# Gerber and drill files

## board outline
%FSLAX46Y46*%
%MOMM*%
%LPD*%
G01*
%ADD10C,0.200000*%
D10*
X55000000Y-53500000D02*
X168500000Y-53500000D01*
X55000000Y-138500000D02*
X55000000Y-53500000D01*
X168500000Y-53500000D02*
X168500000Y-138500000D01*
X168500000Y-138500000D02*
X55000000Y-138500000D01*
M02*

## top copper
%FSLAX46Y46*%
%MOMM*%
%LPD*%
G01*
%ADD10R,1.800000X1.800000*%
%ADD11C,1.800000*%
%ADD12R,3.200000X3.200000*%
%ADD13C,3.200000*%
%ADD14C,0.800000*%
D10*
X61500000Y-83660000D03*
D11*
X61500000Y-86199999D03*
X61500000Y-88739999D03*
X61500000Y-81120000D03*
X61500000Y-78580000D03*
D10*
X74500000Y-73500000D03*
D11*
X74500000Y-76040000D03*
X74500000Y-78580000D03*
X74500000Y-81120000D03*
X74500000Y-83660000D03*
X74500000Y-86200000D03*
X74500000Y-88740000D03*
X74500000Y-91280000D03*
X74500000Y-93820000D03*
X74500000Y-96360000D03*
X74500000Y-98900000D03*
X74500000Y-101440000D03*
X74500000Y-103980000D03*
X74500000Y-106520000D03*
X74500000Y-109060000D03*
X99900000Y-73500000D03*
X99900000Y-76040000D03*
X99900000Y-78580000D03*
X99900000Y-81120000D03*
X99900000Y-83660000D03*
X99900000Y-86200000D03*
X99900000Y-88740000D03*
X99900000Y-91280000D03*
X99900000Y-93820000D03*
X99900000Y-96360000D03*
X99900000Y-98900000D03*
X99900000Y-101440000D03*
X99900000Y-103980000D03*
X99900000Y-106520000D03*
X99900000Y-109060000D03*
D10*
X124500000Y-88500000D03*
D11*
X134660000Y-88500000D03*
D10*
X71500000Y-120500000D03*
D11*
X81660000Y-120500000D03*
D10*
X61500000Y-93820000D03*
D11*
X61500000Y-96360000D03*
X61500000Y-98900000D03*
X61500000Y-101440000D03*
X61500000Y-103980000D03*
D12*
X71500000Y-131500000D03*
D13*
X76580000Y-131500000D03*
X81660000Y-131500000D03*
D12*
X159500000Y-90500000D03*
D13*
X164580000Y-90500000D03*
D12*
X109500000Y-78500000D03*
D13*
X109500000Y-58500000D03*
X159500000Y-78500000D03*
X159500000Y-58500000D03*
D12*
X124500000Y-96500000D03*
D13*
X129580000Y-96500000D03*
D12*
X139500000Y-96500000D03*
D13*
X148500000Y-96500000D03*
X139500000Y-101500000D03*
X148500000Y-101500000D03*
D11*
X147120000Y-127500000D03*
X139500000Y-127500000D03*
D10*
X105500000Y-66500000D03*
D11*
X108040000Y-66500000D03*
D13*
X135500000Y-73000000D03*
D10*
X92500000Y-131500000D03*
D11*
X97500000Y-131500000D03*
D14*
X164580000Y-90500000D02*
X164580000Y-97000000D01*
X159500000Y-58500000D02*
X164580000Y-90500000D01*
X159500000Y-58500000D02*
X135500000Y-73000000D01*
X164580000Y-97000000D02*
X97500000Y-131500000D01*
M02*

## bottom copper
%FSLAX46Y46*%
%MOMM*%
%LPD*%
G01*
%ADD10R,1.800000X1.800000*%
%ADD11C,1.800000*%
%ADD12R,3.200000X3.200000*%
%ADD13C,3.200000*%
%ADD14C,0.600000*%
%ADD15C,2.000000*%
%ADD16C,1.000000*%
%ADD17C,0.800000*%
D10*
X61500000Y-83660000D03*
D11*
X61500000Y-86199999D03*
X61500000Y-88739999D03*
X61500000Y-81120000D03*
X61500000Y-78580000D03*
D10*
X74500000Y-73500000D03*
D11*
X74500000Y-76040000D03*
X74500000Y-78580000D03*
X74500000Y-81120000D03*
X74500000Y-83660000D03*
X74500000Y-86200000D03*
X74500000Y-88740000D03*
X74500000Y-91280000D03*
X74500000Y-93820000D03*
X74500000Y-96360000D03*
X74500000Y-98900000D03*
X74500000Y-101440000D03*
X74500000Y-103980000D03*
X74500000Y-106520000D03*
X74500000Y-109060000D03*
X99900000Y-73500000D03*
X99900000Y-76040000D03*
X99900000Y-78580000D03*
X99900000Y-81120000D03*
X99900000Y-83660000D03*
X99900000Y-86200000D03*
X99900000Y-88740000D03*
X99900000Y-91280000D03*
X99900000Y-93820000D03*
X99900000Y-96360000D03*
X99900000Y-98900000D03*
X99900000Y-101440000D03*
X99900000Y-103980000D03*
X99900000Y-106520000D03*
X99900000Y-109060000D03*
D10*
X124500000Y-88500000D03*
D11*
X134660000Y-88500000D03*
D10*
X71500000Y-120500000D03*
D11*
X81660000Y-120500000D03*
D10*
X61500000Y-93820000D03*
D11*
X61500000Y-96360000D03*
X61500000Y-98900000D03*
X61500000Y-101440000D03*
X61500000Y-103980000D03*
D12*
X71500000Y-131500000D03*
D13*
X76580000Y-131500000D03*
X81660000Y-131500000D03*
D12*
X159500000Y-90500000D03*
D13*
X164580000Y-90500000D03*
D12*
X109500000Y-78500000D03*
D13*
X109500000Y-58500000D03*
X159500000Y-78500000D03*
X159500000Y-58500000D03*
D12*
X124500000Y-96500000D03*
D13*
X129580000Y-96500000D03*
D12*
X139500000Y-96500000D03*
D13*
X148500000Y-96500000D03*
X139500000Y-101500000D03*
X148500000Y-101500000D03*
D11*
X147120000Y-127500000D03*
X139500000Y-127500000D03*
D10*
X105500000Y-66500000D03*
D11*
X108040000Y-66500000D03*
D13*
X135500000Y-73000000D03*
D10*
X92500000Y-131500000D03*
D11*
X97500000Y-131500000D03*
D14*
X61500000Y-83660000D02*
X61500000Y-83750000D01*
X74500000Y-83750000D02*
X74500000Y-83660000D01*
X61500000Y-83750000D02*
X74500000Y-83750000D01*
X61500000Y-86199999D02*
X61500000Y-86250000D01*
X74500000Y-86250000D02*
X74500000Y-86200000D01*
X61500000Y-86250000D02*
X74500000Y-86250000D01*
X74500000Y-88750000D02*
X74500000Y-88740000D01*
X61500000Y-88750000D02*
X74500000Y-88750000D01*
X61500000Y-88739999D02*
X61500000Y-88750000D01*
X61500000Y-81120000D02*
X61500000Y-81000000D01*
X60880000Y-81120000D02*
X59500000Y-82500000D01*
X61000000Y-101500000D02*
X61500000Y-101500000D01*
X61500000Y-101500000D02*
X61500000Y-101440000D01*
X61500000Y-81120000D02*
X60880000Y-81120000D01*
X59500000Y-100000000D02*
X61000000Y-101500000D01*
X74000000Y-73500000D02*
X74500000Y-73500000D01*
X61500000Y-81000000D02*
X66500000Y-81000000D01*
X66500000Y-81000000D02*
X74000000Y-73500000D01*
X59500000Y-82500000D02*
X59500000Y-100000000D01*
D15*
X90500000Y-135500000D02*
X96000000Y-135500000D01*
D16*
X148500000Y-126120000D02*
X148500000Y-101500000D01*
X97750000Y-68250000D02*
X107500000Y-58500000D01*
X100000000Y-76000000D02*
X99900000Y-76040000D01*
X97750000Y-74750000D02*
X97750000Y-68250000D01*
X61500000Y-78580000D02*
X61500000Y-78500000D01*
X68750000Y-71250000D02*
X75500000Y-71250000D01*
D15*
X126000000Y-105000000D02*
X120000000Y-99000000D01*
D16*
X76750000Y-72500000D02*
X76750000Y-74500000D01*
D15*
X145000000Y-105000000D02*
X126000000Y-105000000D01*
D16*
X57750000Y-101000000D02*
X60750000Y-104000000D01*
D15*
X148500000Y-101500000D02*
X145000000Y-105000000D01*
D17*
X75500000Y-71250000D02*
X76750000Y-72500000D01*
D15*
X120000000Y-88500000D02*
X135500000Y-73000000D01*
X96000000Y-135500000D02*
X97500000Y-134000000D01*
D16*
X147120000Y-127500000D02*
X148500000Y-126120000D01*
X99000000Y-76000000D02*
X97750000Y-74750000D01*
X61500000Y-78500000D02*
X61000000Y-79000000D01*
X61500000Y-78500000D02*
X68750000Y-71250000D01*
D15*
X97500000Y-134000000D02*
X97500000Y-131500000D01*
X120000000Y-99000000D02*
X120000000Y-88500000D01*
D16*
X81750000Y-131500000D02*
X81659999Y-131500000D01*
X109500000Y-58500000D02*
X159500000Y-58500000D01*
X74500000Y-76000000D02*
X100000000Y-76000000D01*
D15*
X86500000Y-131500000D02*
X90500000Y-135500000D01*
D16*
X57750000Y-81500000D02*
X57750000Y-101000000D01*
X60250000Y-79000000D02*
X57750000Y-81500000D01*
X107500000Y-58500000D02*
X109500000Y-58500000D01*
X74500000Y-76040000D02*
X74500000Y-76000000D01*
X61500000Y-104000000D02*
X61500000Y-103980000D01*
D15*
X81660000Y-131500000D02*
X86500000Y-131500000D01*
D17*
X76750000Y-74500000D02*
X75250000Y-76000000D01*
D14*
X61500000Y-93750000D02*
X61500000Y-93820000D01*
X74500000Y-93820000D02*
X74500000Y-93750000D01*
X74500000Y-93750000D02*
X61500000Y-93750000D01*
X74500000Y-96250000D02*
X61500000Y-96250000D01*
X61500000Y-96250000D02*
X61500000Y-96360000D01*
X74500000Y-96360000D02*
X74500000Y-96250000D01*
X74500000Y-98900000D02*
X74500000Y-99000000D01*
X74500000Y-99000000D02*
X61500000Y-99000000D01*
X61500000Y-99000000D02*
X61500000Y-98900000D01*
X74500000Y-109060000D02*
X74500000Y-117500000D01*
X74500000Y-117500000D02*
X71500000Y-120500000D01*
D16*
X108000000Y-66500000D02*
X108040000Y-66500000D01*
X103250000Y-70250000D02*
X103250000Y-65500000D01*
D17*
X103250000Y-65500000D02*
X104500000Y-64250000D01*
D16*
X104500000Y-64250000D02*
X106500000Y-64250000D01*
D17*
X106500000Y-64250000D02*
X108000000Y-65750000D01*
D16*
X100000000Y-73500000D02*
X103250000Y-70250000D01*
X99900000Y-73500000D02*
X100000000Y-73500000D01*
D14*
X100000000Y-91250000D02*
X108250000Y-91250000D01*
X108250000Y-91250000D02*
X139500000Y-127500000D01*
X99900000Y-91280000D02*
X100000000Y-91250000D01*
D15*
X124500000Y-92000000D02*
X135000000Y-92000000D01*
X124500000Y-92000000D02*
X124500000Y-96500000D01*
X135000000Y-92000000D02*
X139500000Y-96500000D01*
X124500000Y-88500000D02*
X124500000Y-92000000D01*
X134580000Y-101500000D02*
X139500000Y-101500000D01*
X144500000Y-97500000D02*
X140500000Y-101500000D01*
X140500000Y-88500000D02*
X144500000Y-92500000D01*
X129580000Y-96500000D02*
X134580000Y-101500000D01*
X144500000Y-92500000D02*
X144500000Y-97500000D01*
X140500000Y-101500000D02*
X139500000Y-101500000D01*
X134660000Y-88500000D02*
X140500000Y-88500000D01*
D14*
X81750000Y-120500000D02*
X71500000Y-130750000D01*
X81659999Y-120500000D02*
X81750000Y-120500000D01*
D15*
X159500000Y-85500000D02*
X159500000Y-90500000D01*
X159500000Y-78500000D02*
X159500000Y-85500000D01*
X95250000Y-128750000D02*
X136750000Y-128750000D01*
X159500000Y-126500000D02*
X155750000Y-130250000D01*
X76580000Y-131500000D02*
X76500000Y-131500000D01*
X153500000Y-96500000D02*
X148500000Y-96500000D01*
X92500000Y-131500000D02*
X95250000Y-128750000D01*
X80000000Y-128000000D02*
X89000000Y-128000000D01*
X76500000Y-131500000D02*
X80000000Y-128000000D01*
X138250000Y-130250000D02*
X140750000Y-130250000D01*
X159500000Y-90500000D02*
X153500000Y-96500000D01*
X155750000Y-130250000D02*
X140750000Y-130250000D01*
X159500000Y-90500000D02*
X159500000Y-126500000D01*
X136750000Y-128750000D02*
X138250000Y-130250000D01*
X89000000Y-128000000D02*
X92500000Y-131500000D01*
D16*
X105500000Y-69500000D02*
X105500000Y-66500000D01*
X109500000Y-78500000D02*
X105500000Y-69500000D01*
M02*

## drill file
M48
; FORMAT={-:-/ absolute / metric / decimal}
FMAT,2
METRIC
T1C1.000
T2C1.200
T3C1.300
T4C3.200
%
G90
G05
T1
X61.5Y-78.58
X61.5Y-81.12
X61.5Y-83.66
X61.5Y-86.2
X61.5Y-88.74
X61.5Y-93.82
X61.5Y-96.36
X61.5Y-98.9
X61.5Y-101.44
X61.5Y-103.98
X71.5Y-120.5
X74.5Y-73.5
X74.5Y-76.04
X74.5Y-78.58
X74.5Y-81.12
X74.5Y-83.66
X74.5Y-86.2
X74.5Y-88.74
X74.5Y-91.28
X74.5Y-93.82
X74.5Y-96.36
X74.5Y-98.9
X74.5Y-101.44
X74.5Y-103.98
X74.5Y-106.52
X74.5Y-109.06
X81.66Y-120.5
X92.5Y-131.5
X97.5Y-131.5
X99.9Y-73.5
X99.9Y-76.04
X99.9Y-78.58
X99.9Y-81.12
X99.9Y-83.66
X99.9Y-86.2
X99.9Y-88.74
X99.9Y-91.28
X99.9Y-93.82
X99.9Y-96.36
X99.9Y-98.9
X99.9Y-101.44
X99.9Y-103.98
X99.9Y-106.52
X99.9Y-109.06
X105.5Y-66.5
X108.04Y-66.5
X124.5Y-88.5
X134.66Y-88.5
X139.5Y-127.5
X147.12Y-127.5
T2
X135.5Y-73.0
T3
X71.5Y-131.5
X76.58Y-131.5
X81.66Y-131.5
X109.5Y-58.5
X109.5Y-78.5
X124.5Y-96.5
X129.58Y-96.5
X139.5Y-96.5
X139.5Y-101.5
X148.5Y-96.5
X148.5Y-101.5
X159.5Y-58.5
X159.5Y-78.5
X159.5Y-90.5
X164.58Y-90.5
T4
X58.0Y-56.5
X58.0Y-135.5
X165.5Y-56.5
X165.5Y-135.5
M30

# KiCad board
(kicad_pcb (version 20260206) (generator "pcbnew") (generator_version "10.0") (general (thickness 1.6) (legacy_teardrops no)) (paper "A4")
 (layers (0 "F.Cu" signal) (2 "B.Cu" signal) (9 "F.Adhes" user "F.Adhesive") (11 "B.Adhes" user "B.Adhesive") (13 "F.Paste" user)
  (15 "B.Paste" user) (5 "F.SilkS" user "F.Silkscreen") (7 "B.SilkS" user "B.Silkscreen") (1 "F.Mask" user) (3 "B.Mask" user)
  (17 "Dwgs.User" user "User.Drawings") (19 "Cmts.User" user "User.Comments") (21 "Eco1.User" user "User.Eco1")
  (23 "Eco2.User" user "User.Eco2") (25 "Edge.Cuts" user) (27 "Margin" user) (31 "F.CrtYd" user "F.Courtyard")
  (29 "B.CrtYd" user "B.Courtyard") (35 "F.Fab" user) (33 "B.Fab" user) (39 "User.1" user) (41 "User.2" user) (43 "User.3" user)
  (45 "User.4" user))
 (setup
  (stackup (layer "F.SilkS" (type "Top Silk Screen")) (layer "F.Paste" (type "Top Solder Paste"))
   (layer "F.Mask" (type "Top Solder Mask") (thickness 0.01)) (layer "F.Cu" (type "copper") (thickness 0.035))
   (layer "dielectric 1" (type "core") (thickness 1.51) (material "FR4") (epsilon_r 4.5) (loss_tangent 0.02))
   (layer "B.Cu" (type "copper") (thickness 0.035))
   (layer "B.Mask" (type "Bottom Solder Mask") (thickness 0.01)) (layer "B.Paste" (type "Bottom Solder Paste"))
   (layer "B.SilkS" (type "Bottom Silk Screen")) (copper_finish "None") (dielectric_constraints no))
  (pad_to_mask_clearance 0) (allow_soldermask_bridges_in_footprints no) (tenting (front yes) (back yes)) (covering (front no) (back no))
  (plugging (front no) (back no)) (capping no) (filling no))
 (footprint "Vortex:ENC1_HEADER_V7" (layer "F.Cu") (at 61.5 83.5 -90)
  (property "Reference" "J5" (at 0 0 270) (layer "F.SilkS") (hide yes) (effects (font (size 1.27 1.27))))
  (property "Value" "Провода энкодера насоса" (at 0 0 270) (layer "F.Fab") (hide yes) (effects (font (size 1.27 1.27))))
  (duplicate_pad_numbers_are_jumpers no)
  (pad "1" thru_hole rect (at 0.16 0 270) (size 1.8 1.8) (drill 1) (layers "*.Cu") (remove_unused_layers no) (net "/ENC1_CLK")
   (thermal_bridge_angle 45))
  (pad "2" thru_hole circle (at 2.699999 0 270) (size 1.8 1.8) (drill 1) (layers "*.Cu") (remove_unused_layers no) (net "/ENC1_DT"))
  (pad "3" thru_hole circle (at 5.239999 0 270) (size 1.8 1.8) (drill 1) (layers "*.Cu") (remove_unused_layers no) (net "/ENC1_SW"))
  (pad "4" thru_hole circle (at -2.38 0 270) (size 1.8 1.8) (drill 1) (layers "*.Cu") (remove_unused_layers no) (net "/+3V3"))
  (pad "5" thru_hole circle (at -4.92 0 270) (size 1.8 1.8) (drill 1) (layers "*.Cu") (remove_unused_layers no) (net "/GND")))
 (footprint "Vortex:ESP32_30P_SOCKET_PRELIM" (layer "F.Cu") (at 74.5 73.5)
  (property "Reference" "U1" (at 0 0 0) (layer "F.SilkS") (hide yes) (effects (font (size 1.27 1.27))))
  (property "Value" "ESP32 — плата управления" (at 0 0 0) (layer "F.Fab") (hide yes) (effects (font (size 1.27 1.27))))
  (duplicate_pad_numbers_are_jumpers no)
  (pad "1" thru_hole rect (at 0 0) (size 1.8 1.8) (drill 1) (layers "*.Cu") (remove_unused_layers no) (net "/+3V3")
   (thermal_bridge_angle 45))
  (pad "2" thru_hole circle (at 0 2.54) (size 1.8 1.8) (drill 1) (layers "*.Cu") (remove_unused_layers no) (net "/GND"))
  (pad "3" thru_hole circle (at 0 5.08) (size 1.8 1.8) (drill 1) (layers "*.Cu") (remove_unused_layers no) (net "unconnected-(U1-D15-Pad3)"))
  (pad "4" thru_hole circle (at 0 7.62) (size 1.8 1.8) (drill 1) (layers "*.Cu") (remove_unused_layers no) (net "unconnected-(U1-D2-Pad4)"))
  (pad "5" thru_hole circle (at 0 10.16) (size 1.8 1.8) (drill 1) (layers "*.Cu") (remove_unused_layers no) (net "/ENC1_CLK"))
  (pad "6" thru_hole circle (at 0 12.7) (size 1.8 1.8) (drill 1) (layers "*.Cu") (remove_unused_layers no) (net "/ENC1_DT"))
  (pad "7" thru_hole circle (at 0 15.24) (size 1.8 1.8) (drill 1) (layers "*.Cu") (remove_unused_layers no) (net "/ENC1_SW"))
  (pad "8" thru_hole circle (at 0 17.78) (size 1.8 1.8) (drill 1) (layers "*.Cu") (remove_unused_layers no) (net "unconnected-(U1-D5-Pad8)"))
  (pad "9" thru_hole circle (at 0 20.32) (size 1.8 1.8) (drill 1) (layers "*.Cu") (remove_unused_layers no) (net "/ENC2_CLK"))
  (pad "10" thru_hole circle (at 0 22.86) (size 1.8 1.8) (drill 1) (layers "*.Cu") (remove_unused_layers no) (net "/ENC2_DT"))
  (pad "11" thru_hole circle (at 0 25.4) (size 1.8 1.8) (drill 1) (layers "*.Cu") (remove_unused_layers no) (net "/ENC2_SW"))
  (pad "12" thru_hole circle (at 0 27.94) (size 1.8 1.8) (drill 1) (layers "*.Cu") (remove_unused_layers no)
   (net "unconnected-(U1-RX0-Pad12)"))
  (pad "13" thru_hole circle (at 0 30.48) (size 1.8 1.8) (drill 1) (layers "*.Cu") (remove_unused_layers no)
   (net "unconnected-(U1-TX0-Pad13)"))
  (pad "14" thru_hole circle (at 0 33.02) (size 1.8 1.8) (drill 1) (layers "*.Cu") (remove_unused_layers no)
   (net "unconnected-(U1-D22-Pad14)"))
  (pad "15" thru_hole circle (at 0 35.56) (size 1.8 1.8) (drill 1) (layers "*.Cu") (remove_unused_layers no) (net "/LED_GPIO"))
  (pad "16" thru_hole circle (at 25.4 0) (size 1.8 1.8) (drill 1) (layers "*.Cu") (remove_unused_layers no) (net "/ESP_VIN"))
  (pad "17" thru_hole circle (at 25.4 2.54) (size 1.8 1.8) (drill 1) (layers "*.Cu") (remove_unused_layers no) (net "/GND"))
  (pad "18" thru_hole circle (at 25.4 5.08) (size 1.8 1.8) (drill 1) (layers "*.Cu") (remove_unused_layers no)
   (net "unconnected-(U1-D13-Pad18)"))
  (pad "19" thru_hole circle (at 25.4 7.62) (size 1.8 1.8) (drill 1) (layers "*.Cu") (remove_unused_layers no)
   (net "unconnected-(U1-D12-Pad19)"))
  (pad "20" thru_hole circle (at 25.4 10.16) (size 1.8 1.8) (drill 1) (layers "*.Cu") (remove_unused_layers no)
   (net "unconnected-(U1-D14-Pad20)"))
  (pad "21" thru_hole circle (at 25.4 12.7) (size 1.8 1.8) (drill 1) (layers "*.Cu") (remove_unused_layers no)
   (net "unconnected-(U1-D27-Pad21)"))
  (pad "22" thru_hole circle (at 25.4 15.24) (size 1.8 1.8) (drill 1) (layers "*.Cu") (remove_unused_layers no)
   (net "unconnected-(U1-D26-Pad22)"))
  (pad "23" thru_hole circle (at 25.4 17.78) (size 1.8 1.8) (drill 1) (layers "*.Cu") (remove_unused_layers no) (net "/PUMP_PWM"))
  (pad "24" thru_hole circle (at 25.4 20.32) (size 1.8 1.8) (drill 1) (layers "*.Cu") (remove_unused_layers no)
   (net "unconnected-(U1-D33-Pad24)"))
  (pad "25" thru_hole circle (at 25.4 22.86) (size 1.8 1.8) (drill 1) (layers "*.Cu") (remove_unused_layers no)
   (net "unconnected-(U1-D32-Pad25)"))
  (pad "26" thru_hole circle (at 25.4 25.4) (size 1.8 1.8) (drill 1) (layers "*.Cu") (remove_unused_layers no)
   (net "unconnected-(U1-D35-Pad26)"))
  (pad "27" thru_hole circle (at 25.4 27.94) (size 1.8 1.8) (drill 1) (layers "*.Cu") (remove_unused_layers no)
   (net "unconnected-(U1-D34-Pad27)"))
  (pad "28" thru_hole circle (at 25.4 30.48) (size 1.8 1.8) (drill 1) (layers "*.Cu") (remove_unused_layers no)
   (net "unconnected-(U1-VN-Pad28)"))
  (pad "29" thru_hole circle (at 25.4 33.02) (size 1.8 1.8) (drill 1) (layers "*.Cu") (remove_unused_layers no)
   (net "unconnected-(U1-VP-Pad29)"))
  (pad "30" thru_hole circle (at 25.4 35.56) (size 1.8 1.8) (drill 1) (layers "*.Cu") (remove_unused_layers no)
   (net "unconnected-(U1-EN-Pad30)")))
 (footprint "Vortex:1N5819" (layer "F.Cu") (at 124.5 88.5)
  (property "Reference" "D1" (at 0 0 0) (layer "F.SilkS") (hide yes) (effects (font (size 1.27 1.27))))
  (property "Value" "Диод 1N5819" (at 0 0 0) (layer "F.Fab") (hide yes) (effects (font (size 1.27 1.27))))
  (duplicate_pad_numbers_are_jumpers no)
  (pad "1" thru_hole rect (at 0 0) (size 1.8 1.8) (drill 1) (layers "*.Cu") (remove_unused_layers no) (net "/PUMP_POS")
   (thermal_bridge_angle 45))
  (pad "2" thru_hole circle (at 10.16 0) (size 1.8 1.8) (drill 1) (layers "*.Cu") (remove_unused_layers no) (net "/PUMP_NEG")))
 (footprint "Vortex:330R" (layer "F.Cu") (at 71.5 120.5)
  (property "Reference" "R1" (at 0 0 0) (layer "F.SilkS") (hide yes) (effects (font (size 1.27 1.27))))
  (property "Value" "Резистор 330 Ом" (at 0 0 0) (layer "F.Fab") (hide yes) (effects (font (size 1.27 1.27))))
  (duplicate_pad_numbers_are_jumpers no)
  (pad "1" thru_hole rect (at 0 0) (size 1.8 1.8) (drill 1) (layers "*.Cu") (remove_unused_layers no) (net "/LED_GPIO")
   (thermal_bridge_angle 45))
  (pad "2" thru_hole circle (at 10.16 0) (size 1.8 1.8) (drill 1) (layers "*.Cu") (remove_unused_layers no) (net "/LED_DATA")))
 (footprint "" (layer "F.Cu") (at 58 135.5)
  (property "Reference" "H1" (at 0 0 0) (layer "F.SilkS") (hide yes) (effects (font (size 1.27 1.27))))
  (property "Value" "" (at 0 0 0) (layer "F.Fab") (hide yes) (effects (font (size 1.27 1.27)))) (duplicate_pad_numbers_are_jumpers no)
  (pad "" np_thru_hole circle (at 0 0) (size 3.2 3.2) (drill 3.2) (layers "*.Cu")))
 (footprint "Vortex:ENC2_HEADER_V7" (layer "F.Cu") (at 61.5 96.5 -90)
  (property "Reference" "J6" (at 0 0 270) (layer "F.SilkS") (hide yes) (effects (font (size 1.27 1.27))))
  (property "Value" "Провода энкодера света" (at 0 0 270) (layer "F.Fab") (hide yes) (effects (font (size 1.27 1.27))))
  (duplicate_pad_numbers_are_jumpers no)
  (pad "1" thru_hole rect (at -2.68 0 270) (size 1.8 1.8) (drill 1) (layers "*.Cu") (remove_unused_layers no) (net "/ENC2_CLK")
   (thermal_bridge_angle 45))
  (pad "2" thru_hole circle (at -0.14 0 270) (size 1.8 1.8) (drill 1) (layers "*.Cu") (remove_unused_layers no) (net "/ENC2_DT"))
  (pad "3" thru_hole circle (at 2.4 0 270) (size 1.8 1.8) (drill 1) (layers "*.Cu") (remove_unused_layers no) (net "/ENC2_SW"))
  (pad "4" thru_hole circle (at 4.94 0 270) (size 1.8 1.8) (drill 1) (layers "*.Cu") (remove_unused_layers no) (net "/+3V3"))
  (pad "5" thru_hole circle (at 7.48 0 270) (size 1.8 1.8) (drill 1) (layers "*.Cu") (remove_unused_layers no) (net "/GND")))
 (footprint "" (layer "F.Cu") (at 58 56.5)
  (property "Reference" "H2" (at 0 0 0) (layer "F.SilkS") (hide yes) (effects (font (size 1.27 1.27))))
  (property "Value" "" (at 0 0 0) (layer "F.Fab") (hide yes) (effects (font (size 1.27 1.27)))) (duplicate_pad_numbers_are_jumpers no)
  (pad "" np_thru_hole circle (at 0 0) (size 3.2 3.2) (drill 3.2) (layers "*.Cu")))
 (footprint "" (layer "F.Cu") (at 165.5 135.5)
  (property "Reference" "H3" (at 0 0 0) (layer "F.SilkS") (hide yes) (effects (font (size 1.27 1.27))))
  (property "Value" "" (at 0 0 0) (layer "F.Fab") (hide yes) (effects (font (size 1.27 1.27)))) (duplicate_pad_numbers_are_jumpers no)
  (pad "" np_thru_hole circle (at 0 0) (size 3.2 3.2) (drill 3.2) (layers "*.Cu")))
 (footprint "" (layer "F.Cu") (at 165.5 56.5)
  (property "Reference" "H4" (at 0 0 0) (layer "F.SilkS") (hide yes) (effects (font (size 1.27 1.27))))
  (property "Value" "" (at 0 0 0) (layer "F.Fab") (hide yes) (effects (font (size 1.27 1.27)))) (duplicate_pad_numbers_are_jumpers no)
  (pad "" np_thru_hole circle (at 0 0) (size 3.2 3.2) (drill 3.2) (layers "*.Cu")))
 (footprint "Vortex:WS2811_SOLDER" (layer "F.Cu") (at 71.5 131.5)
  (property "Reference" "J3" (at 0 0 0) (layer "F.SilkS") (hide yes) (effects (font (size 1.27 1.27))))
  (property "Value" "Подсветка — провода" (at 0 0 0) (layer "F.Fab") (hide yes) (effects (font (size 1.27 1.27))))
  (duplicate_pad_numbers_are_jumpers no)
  (pad "1" thru_hole rect (at 0 0) (size 3.2 3.2) (drill 1.3) (layers "*.Cu") (remove_unused_layers no) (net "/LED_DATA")
   (thermal_bridge_angle 45))
  (pad "2" thru_hole circle (at 5.08 0) (size 3.2 3.2) (drill 1.3) (layers "*.Cu") (remove_unused_layers no) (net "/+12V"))
  (pad "3" thru_hole circle (at 10.16 0) (size 3.2 3.2) (drill 1.3) (layers "*.Cu") (remove_unused_layers no) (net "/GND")))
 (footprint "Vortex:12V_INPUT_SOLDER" (layer "F.Cu") (at 159.5 90.5)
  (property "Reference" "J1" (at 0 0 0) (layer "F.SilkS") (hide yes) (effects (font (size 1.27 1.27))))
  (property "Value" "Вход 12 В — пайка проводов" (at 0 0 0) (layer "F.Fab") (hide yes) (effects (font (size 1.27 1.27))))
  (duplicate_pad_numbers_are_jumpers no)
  (pad "1" thru_hole rect (at 0 0) (size 3.2 3.2) (drill 1.3) (layers "*.Cu") (remove_unused_layers no) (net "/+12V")
   (thermal_bridge_angle 45))
  (pad "2" thru_hole circle (at 5.08 0) (size 3.2 3.2) (drill 1.3) (layers "*.Cu") (remove_unused_layers no) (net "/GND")))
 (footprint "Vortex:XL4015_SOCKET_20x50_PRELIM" (layer "F.Cu") (at 109.5 78.5 90)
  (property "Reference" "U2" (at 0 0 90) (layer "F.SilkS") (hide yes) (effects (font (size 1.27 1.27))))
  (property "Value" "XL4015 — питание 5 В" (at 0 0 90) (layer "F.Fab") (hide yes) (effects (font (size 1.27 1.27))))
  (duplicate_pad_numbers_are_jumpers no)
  (pad "1" thru_hole rect (at 0 0 90) (size 3.2 3.2) (drill 1.3) (layers "*.Cu") (remove_unused_layers no) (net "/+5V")
   (thermal_bridge_angle 45))
  (pad "2" thru_hole circle (at 20 0 90) (size 3.2 3.2) (drill 1.3) (layers "*.Cu") (remove_unused_layers no) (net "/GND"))
  (pad "3" thru_hole circle (at 0 50 90) (size 3.2 3.2) (drill 1.3) (layers "*.Cu") (remove_unused_layers no) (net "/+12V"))
  (pad "4" thru_hole circle (at 20 50 90) (size 3.2 3.2) (drill 1.3) (layers "*.Cu") (remove_unused_layers no) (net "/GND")))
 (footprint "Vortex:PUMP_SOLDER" (layer "F.Cu") (at 124.5 96.5)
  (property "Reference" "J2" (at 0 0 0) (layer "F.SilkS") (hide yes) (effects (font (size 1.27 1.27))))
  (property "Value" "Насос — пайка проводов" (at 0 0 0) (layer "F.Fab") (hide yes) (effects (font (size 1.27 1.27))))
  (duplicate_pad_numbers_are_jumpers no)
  (pad "1" thru_hole rect (at 0 0) (size 3.2 3.2) (drill 1.3) (layers "*.Cu") (remove_unused_layers no) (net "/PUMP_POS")
   (thermal_bridge_angle 45))
  (pad "2" thru_hole circle (at 5.08 0) (size 3.2 3.2) (drill 1.3) (layers "*.Cu") (remove_unused_layers no) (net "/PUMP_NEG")))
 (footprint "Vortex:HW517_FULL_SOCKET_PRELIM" (layer "F.Cu") (at 139.5 96.5)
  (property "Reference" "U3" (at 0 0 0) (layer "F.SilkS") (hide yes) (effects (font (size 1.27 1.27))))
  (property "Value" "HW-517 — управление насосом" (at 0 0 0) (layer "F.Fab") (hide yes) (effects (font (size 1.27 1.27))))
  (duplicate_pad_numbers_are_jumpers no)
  (pad "1" thru_hole rect (at 0 0) (size 3.2 3.2) (drill 1.3) (layers "*.Cu") (remove_unused_layers no) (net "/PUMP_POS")
   (thermal_bridge_angle 45))
  (pad "2" thru_hole circle (at 9 0) (size 3.2 3.2) (drill 1.3) (layers "*.Cu") (remove_unused_layers no) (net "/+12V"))
  (pad "3" thru_hole circle (at 0 5) (size 3.2 3.2) (drill 1.3) (layers "*.Cu") (remove_unused_layers no) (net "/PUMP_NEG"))
  (pad "4" thru_hole circle (at 9 5) (size 3.2 3.2) (drill 1.3) (layers "*.Cu") (remove_unused_layers no) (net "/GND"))
  (pad "5" thru_hole circle (at 7.62 31) (size 1.8 1.8) (drill 1) (layers "*.Cu") (remove_unused_layers no) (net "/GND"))
  (pad "6" thru_hole circle (at 0 31) (size 1.8 1.8) (drill 1) (layers "*.Cu") (remove_unused_layers no) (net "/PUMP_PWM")))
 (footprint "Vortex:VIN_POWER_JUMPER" (layer "F.Cu") (at 105.5 66.5)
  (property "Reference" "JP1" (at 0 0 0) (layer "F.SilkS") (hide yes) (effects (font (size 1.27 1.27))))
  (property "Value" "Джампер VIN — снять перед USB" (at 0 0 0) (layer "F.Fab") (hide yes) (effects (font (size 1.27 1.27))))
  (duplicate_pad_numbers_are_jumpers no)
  (pad "1" thru_hole rect (at 0 0) (size 1.8 1.8) (drill 1) (layers "*.Cu") (remove_unused_layers no) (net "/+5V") (thermal_bridge_angle 45))
  (pad "2" thru_hole circle (at 2.54 0) (size 1.8 1.8) (drill 1) (layers "*.Cu") (remove_unused_layers no) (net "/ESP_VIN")))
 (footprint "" (layer "F.Cu") (at 135.5 73)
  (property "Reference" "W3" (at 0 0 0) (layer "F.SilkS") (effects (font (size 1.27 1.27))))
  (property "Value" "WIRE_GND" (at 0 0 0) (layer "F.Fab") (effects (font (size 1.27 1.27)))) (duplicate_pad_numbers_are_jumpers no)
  (pad "1" thru_hole circle (at 0 0) (size 3.2 3.2) (drill 1.2) (layers "*.Cu") (remove_unused_layers no) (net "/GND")))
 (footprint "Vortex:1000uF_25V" (layer "F.Cu") (at 92.5 131.5)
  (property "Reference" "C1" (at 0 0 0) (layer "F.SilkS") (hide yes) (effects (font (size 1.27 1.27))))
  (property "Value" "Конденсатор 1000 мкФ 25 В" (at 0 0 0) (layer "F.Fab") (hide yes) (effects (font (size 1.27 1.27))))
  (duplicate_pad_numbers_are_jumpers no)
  (pad "1" thru_hole rect (at 0 0) (size 1.8 1.8) (drill 1) (layers "*.Cu") (remove_unused_layers no) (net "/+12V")
   (thermal_bridge_angle 45))
  (pad "2" thru_hole circle (at 5 0) (size 1.8 1.8) (drill 1) (layers "*.Cu") (remove_unused_layers no) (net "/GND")))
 (gr_line (start 55 53.5) (end 168.5 53.5) (stroke (width 0.2) (type default)) (layer "Edge.Cuts"))
 (gr_line (start 55 138.5) (end 55 53.5) (stroke (width 0.2) (type default)) (layer "Edge.Cuts"))
 (gr_line (start 168.5 53.5) (end 168.5 138.5) (stroke (width 0.2) (type default)) (layer "Edge.Cuts"))
 (gr_line (start 168.5 138.5) (end 55 138.5) (stroke (width 0.2) (type default)) (layer "Edge.Cuts"))
 (segment (start 61.5 83.66) (end 61.5 83.75) (width 0.6) (layer "B.Cu") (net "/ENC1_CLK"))
 (segment (start 74.5 83.75) (end 74.5 83.66) (width 0.6) (layer "B.Cu") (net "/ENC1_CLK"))
 (segment (start 61.5 83.75) (end 74.5 83.75) (width 0.6) (layer "B.Cu") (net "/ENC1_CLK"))
 (segment (start 61.5 86.199999) (end 61.5 86.25) (width 0.6) (layer "B.Cu") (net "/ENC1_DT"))
 (segment (start 74.5 86.25) (end 74.5 86.2) (width 0.6) (layer "B.Cu") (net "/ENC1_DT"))
 (segment (start 61.5 86.25) (end 74.5 86.25) (width 0.6) (layer "B.Cu") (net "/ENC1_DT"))
 (segment (start 74.5 88.75) (end 74.5 88.74) (width 0.6) (layer "B.Cu") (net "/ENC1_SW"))
 (segment (start 61.5 88.75) (end 74.5 88.75) (width 0.6) (layer "B.Cu") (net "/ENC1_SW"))
 (segment (start 61.5 88.739999) (end 61.5 88.75) (width 0.6) (layer "B.Cu") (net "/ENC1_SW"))
 (segment (start 61.5 81.12) (end 61.5 81) (width 0.6) (layer "B.Cu") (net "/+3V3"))
 (segment (start 60.88 81.12) (end 59.5 82.5) (width 0.6) (layer "B.Cu") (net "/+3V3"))
 (segment (start 61 101.5) (end 61.5 101.5) (width 0.6) (layer "B.Cu") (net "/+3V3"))
 (segment (start 61.5 101.5) (end 61.5 101.44) (width 0.6) (layer "B.Cu") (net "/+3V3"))
 (segment (start 61.5 81.12) (end 60.88 81.12) (width 0.6) (layer "B.Cu") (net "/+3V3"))
 (segment (start 59.5 100) (end 61 101.5) (width 0.6) (layer "B.Cu") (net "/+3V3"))
 (segment (start 74 73.5) (end 74.5 73.5) (width 0.6) (layer "B.Cu") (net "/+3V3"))
 (segment (start 61.5 81) (end 66.5 81) (width 0.6) (layer "B.Cu") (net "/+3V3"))
 (segment (start 66.5 81) (end 74 73.5) (width 0.6) (layer "B.Cu") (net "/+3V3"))
 (segment (start 59.5 82.5) (end 59.5 100) (width 0.6) (layer "B.Cu") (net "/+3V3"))
 (segment (start 164.58 90.5) (end 164.58 97) (width 0.8) (layer "F.Cu") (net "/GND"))
 (segment (start 159.5 58.5) (end 164.58 90.5) (width 0.8) (layer "F.Cu") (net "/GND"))
 (segment (start 159.5 58.5) (end 135.5 73) (width 0.8) (layer "F.Cu") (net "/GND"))
 (segment (start 164.58 97) (end 97.5 131.5) (width 0.8) (layer "F.Cu") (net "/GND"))
 (segment (start 90.5 135.5) (end 96 135.5) (width 2) (layer "B.Cu") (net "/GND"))
 (segment (start 148.5 126.12) (end 148.5 101.5) (width 1) (layer "B.Cu") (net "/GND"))
 (segment (start 97.75 68.25) (end 107.5 58.5) (width 1) (layer "B.Cu") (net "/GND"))
 (segment (start 100 76) (end 99.9 76.04) (width 1) (layer "B.Cu") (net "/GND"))
 (segment (start 97.75 74.75) (end 97.75 68.25) (width 1) (layer "B.Cu") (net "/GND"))
 (segment (start 61.5 78.58) (end 61.5 78.5) (width 1) (layer "B.Cu") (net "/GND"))
 (segment (start 68.75 71.25) (end 75.5 71.25) (width 1) (layer "B.Cu") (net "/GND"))
 (segment (start 126 105) (end 120 99) (width 2) (layer "B.Cu") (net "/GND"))
 (segment (start 76.75 72.5) (end 76.75 74.5) (width 1) (layer "B.Cu") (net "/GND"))
 (segment (start 145 105) (end 126 105) (width 2) (layer "B.Cu") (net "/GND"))
 (segment (start 57.75 101) (end 60.75 104) (width 1) (layer "B.Cu") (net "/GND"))
 (segment (start 148.5 101.5) (end 145 105) (width 2) (layer "B.Cu") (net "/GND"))
 (segment (start 75.5 71.25) (end 76.75 72.5) (width 0.8) (layer "B.Cu") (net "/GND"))
 (segment (start 120 88.5) (end 135.5 73) (width 2) (layer "B.Cu") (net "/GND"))
 (segment (start 96 135.5) (end 97.5 134) (width 2) (layer "B.Cu") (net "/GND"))
 (segment (start 147.12 127.5) (end 148.5 126.12) (width 1) (layer "B.Cu") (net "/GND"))
 (segment (start 99 76) (end 97.75 74.75) (width 1) (layer "B.Cu") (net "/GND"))
 (segment (start 61.5 78.5) (end 61 79) (width 1) (layer "B.Cu") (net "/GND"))
 (segment (start 61.5 78.5) (end 68.75 71.25) (width 1) (layer "B.Cu") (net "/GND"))
 (segment (start 97.5 134) (end 97.5 131.5) (width 2) (layer "B.Cu") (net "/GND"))
 (segment (start 120 99) (end 120 88.5) (width 2) (layer "B.Cu") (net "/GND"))
 (segment (start 81.75 131.5) (end 81.659999 131.5) (width 1) (layer "B.Cu") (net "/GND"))
 (segment (start 109.5 58.5) (end 159.5 58.5) (width 1) (layer "B.Cu") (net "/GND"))
 (segment (start 74.5 76) (end 100 76) (width 1) (layer "B.Cu") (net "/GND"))
 (segment (start 86.5 131.5) (end 90.5 135.5) (width 2) (layer "B.Cu") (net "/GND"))
 (segment (start 57.75 81.5) (end 57.75 101) (width 1) (layer "B.Cu") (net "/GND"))
 (segment (start 60.25 79) (end 57.75 81.5) (width 1) (layer "B.Cu") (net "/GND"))
 (segment (start 107.5 58.5) (end 109.5 58.5) (width 1) (layer "B.Cu") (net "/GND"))
 (segment (start 74.5 76.04) (end 74.5 76) (width 1) (layer "B.Cu") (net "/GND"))
 (segment (start 61.5 104) (end 61.5 103.98) (width 1) (layer "B.Cu") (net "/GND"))
 (segment (start 81.66 131.5) (end 86.5 131.5) (width 2) (layer "B.Cu") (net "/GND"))
 (segment (start 76.75 74.5) (end 75.25 76) (width 0.8) (layer "B.Cu") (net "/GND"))
 (segment (start 61.5 93.75) (end 61.5 93.82) (width 0.6) (layer "B.Cu") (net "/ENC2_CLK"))
 (segment (start 74.5 93.82) (end 74.5 93.75) (width 0.6) (layer "B.Cu") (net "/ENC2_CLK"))
 (segment (start 74.5 93.75) (end 61.5 93.75) (width 0.6) (layer "B.Cu") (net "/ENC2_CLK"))
 (segment (start 74.5 96.25) (end 61.5 96.25) (width 0.6) (layer "B.Cu") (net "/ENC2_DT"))
 (segment (start 61.5 96.25) (end 61.5 96.36) (width 0.6) (layer "B.Cu") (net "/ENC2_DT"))
 (segment (start 74.5 96.36) (end 74.5 96.25) (width 0.6) (layer "B.Cu") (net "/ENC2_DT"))
 (segment (start 74.5 98.9) (end 74.5 99) (width 0.6) (layer "B.Cu") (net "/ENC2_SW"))
 (segment (start 74.5 99) (end 61.5 99) (width 0.6) (layer "B.Cu") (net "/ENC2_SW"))
 (segment (start 61.5 99) (end 61.5 98.9) (width 0.6) (layer "B.Cu") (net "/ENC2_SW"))
 (segment (start 74.5 109.06) (end 74.5 117.5) (width 0.6) (layer "B.Cu") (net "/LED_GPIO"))
 (segment (start 74.5 117.5) (end 71.5 120.5) (width 0.6) (layer "B.Cu") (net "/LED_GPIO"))
 (segment (start 108 66.5) (end 108.04 66.5) (width 1) (layer "B.Cu") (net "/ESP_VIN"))
 (segment (start 103.25 70.25) (end 103.25 65.5) (width 1) (layer "B.Cu") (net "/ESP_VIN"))
 (segment (start 103.25 65.5) (end 104.5 64.25) (width 0.8) (layer "B.Cu") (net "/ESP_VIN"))
 (segment (start 104.5 64.25) (end 106.5 64.25) (width 1) (layer "B.Cu") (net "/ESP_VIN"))
 (segment (start 106.5 64.25) (end 108 65.75) (width 0.8) (layer "B.Cu") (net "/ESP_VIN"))
 (segment (start 100 73.5) (end 103.25 70.25) (width 1) (layer "B.Cu") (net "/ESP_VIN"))
 (segment (start 99.9 73.5) (end 100 73.5) (width 1) (layer "B.Cu") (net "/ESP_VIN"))
 (segment (start 100 91.25) (end 108.25 91.25) (width 0.6) (layer "B.Cu") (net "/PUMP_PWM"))
 (segment (start 108.25 91.25) (end 139.5 127.5) (width 0.6) (layer "B.Cu") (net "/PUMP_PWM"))
 (segment (start 99.9 91.28) (end 100 91.25) (width 0.6) (layer "B.Cu") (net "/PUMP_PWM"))
 (segment (start 124.5 92) (end 135 92) (width 2) (layer "B.Cu") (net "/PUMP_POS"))
 (segment (start 124.5 92) (end 124.5 96.5) (width 2) (layer "B.Cu") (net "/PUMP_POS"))
 (segment (start 135 92) (end 139.5 96.5) (width 2) (layer "B.Cu") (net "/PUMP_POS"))
 (segment (start 124.5 88.5) (end 124.5 92) (width 2) (layer "B.Cu") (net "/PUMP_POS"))
 (segment (start 134.58 101.5) (end 139.5 101.5) (width 2) (layer "B.Cu") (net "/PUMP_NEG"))
 (segment (start 144.5 97.5) (end 140.5 101.5) (width 2) (layer "B.Cu") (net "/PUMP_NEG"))
 (segment (start 140.5 88.5) (end 144.5 92.5) (width 2) (layer "B.Cu") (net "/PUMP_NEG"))
 (segment (start 129.58 96.5) (end 134.58 101.5) (width 2) (layer "B.Cu") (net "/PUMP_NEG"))
 (segment (start 144.5 92.5) (end 144.5 97.5) (width 2) (layer "B.Cu") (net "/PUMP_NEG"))
 (segment (start 140.5 101.5) (end 139.5 101.5) (width 2) (layer "B.Cu") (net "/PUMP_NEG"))
 (segment (start 134.66 88.5) (end 140.5 88.5) (width 2) (layer "B.Cu") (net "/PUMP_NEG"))
 (segment (start 81.75 120.5) (end 71.5 130.75) (width 0.6) (layer "B.Cu") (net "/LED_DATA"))
 (segment (start 81.659999 120.5) (end 81.75 120.5) (width 0.6) (layer "B.Cu") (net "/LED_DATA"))
 (segment (start 159.5 85.5) (end 159.5 90.5) (width 2) (layer "B.Cu") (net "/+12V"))
 (segment (start 159.5 78.5) (end 159.5 85.5) (width 2) (layer "B.Cu") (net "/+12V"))
 (segment (start 95.25 128.75) (end 136.75 128.75) (width 2) (layer "B.Cu") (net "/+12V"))
 (segment (start 159.5 126.5) (end 155.75 130.25) (width 2) (layer "B.Cu") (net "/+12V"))
 (segment (start 76.58 131.5) (end 76.5 131.5) (width 2) (layer "B.Cu") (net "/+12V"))
 (segment (start 153.5 96.5) (end 148.5 96.5) (width 2) (layer "B.Cu") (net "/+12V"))
 (segment (start 92.5 131.5) (end 95.25 128.75) (width 2) (layer "B.Cu") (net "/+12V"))
 (segment (start 80 128) (end 89 128) (width 2) (layer "B.Cu") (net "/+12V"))
 (segment (start 76.5 131.5) (end 80 128) (width 2) (layer "B.Cu") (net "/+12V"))
 (segment (start 138.25 130.25) (end 140.75 130.25) (width 2) (layer "B.Cu") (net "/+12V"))
 (segment (start 159.5 90.5) (end 153.5 96.5) (width 2) (layer "B.Cu") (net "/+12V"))
 (segment (start 155.75 130.25) (end 140.75 130.25) (width 2) (layer "B.Cu") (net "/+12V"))
 (segment (start 159.5 90.5) (end 159.5 126.5) (width 2) (layer "B.Cu") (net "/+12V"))
 (segment (start 136.75 128.75) (end 138.25 130.25) (width 2) (layer "B.Cu") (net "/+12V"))
 (segment (start 89 128) (end 92.5 131.5) (width 2) (layer "B.Cu") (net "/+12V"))
 (segment (start 105.5 69.5) (end 105.5 66.5) (width 1) (layer "B.Cu") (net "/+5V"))
 (segment (start 109.5 78.5) (end 105.5 69.5) (width 1) (layer "B.Cu") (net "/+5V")))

